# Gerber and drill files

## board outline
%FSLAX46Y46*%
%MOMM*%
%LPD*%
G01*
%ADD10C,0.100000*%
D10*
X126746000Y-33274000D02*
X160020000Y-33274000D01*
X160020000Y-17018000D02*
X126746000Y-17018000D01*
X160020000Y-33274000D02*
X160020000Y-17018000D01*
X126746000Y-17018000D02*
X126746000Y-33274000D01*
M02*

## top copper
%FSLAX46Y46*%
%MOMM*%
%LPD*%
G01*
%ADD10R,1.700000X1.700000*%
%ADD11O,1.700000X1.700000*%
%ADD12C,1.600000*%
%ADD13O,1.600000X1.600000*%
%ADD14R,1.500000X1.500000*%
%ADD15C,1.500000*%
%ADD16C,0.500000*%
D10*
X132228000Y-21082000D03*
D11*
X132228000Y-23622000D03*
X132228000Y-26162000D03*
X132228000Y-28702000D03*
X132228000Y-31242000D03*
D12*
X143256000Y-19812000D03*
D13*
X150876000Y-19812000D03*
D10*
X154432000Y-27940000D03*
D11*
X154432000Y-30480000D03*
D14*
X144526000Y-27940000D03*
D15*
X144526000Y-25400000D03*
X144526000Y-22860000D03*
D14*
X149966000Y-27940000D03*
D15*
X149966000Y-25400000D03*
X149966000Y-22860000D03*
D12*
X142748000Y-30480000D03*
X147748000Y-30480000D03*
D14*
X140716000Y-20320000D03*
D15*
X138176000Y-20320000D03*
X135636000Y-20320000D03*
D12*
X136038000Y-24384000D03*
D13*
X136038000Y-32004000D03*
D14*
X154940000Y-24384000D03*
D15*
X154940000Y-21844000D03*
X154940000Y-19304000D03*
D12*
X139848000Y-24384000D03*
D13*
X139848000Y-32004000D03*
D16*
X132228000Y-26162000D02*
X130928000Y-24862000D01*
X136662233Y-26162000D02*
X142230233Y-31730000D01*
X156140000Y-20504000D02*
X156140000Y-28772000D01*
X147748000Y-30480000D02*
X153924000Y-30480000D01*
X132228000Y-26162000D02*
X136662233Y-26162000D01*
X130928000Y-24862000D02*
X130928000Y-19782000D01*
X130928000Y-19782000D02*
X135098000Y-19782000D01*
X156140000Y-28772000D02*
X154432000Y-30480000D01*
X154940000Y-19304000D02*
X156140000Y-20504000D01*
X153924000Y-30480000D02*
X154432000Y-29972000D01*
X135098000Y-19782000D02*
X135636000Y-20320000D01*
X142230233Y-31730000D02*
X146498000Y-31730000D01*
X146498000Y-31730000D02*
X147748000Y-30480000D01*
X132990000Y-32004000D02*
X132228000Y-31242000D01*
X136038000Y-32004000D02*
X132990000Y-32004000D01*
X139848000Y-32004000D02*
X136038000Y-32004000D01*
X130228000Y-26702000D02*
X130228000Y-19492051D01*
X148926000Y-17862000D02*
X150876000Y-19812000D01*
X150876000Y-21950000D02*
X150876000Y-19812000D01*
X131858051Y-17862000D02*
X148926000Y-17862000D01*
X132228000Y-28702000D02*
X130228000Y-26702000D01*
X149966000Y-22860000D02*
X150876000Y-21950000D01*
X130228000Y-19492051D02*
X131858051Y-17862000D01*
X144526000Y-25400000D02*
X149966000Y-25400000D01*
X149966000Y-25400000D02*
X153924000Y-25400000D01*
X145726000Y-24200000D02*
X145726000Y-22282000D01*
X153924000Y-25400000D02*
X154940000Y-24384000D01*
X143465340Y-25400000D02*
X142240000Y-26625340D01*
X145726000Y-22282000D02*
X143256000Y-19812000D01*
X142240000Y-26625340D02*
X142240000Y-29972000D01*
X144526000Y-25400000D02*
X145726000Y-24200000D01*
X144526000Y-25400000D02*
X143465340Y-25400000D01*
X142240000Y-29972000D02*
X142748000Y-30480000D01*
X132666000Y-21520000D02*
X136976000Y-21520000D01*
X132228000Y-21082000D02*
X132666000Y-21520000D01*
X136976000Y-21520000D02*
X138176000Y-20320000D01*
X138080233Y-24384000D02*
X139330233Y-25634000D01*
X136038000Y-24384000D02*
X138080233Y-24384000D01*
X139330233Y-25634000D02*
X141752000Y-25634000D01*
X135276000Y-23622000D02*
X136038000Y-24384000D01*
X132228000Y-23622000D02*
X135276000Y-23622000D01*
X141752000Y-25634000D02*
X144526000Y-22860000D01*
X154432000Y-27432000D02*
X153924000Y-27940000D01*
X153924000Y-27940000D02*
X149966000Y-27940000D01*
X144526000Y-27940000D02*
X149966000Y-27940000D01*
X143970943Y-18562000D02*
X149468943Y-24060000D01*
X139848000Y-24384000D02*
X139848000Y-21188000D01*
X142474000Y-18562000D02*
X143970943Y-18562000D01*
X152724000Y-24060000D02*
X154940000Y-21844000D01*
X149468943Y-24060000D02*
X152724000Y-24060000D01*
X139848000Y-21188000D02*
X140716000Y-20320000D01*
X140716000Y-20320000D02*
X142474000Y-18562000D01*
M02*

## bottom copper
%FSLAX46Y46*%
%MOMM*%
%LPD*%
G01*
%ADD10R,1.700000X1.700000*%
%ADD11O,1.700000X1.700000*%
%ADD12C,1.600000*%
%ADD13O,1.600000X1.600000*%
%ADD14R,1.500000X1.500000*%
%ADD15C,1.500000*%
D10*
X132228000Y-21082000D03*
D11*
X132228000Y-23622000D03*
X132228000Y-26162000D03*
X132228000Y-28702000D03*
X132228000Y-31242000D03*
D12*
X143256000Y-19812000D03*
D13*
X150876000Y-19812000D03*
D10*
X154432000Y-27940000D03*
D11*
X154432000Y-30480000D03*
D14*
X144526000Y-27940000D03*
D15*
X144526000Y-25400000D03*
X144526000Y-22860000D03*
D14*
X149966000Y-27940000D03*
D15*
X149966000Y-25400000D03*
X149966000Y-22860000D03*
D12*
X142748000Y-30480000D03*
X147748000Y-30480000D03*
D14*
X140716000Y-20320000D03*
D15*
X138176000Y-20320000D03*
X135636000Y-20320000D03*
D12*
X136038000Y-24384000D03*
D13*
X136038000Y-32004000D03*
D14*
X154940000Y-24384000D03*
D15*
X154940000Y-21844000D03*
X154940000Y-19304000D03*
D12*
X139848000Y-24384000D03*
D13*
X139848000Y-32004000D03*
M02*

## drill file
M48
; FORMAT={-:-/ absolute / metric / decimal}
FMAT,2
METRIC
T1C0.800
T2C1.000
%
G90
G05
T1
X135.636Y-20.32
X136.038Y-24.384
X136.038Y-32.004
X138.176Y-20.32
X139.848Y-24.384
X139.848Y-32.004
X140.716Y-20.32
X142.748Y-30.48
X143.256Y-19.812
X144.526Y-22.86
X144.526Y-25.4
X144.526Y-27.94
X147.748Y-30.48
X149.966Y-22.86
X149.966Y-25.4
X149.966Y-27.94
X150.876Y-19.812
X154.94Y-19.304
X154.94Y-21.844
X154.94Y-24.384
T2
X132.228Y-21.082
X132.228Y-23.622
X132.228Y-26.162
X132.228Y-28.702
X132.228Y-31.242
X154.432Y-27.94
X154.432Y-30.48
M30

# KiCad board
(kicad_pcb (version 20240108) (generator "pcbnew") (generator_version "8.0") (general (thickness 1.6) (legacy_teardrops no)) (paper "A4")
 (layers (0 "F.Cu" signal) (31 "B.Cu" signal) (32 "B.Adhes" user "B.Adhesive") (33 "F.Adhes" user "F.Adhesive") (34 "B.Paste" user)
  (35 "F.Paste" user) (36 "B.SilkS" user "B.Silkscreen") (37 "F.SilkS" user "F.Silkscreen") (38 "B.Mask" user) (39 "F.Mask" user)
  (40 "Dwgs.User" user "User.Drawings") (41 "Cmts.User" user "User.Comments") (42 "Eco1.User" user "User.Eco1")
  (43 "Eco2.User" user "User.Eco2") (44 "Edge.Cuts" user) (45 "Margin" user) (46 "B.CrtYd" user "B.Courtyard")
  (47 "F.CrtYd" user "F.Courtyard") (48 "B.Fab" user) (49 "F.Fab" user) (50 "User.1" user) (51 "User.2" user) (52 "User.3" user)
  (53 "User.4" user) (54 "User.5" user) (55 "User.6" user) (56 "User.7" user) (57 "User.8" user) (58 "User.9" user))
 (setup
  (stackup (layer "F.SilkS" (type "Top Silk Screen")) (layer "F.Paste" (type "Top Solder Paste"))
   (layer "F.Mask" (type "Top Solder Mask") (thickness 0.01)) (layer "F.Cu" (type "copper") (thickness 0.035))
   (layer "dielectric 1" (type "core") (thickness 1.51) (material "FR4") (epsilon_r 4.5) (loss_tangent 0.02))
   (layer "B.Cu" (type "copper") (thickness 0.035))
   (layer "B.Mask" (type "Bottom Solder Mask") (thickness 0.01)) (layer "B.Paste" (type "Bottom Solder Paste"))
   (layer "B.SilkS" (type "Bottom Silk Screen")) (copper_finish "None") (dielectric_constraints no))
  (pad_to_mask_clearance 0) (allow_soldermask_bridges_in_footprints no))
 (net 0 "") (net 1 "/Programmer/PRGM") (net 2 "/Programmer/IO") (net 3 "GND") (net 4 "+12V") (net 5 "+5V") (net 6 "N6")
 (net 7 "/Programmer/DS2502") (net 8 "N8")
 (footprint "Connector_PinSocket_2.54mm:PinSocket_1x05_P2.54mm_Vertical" (layer "F.Cu") (at 132.228 21.082)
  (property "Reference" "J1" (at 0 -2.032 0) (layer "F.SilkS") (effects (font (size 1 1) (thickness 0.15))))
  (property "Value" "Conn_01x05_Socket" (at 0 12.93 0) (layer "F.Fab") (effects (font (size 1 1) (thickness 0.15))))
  (pad "1" thru_hole rect (at 0 0) (size 1.7 1.7) (drill 1) (layers "*.Cu" "*.Mask") (remove_unused_layers no) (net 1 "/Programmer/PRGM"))
  (pad "2" thru_hole oval (at 0 2.54) (size 1.7 1.7) (drill 1) (layers "*.Cu" "*.Mask") (remove_unused_layers no) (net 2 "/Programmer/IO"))
  (pad "3" thru_hole oval (at 0 5.08) (size 1.7 1.7) (drill 1) (layers "*.Cu" "*.Mask") (remove_unused_layers no) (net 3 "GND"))
  (pad "4" thru_hole oval (at 0 7.62) (size 1.7 1.7) (drill 1) (layers "*.Cu" "*.Mask") (remove_unused_layers no) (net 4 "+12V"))
  (pad "5" thru_hole oval (at 0 10.16) (size 1.7 1.7) (drill 1) (layers "*.Cu" "*.Mask") (remove_unused_layers no) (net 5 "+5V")))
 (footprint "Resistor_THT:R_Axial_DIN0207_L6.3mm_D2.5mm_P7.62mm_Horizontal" (layer "F.Cu") (at 143.256 19.812)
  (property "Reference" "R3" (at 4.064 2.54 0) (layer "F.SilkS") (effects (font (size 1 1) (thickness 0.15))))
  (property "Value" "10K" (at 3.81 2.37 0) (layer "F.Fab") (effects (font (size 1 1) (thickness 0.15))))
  (pad "1" thru_hole circle (at 0 0) (size 1.6 1.6) (drill 0.8) (layers "*.Cu" "*.Mask") (remove_unused_layers no) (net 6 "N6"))
  (pad "2" thru_hole oval (at 7.62 0) (size 1.6 1.6) (drill 0.8) (layers "*.Cu" "*.Mask") (remove_unused_layers no) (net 4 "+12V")))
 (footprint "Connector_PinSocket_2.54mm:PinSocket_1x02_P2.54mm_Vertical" (layer "F.Cu") (at 154.432 27.94)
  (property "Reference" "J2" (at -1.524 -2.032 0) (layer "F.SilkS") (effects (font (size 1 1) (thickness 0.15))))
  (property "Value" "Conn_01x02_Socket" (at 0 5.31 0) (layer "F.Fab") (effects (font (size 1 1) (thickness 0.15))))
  (pad "1" thru_hole rect (at 0 0) (size 1.7 1.7) (drill 1) (layers "*.Cu" "*.Mask") (remove_unused_layers no) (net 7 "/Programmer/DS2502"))
  (pad "2" thru_hole oval (at 0 2.54) (size 1.7 1.7) (drill 1) (layers "*.Cu" "*.Mask") (remove_unused_layers no) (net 3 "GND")))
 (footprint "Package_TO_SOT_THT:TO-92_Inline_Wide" (layer "F.Cu") (at 144.526 27.94 90)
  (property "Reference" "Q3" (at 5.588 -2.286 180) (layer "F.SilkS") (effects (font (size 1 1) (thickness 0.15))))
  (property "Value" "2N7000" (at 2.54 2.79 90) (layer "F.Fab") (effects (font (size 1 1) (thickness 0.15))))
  (pad "1" thru_hole rect (at 0 0 90) (size 1.5 1.5) (drill 0.8) (layers "*.Cu" "*.Mask") (remove_unused_layers no)
   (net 7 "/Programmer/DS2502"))
  (pad "2" thru_hole circle (at 2.54 0 90) (size 1.5 1.5) (drill 0.8) (layers "*.Cu" "*.Mask") (remove_unused_layers no) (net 6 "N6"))
  (pad "3" thru_hole circle (at 5.08 0 90) (size 1.5 1.5) (drill 0.8) (layers "*.Cu" "*.Mask") (remove_unused_layers no)
   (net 2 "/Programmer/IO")))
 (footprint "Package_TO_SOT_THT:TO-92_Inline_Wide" (layer "F.Cu") (at 149.966 27.94 90)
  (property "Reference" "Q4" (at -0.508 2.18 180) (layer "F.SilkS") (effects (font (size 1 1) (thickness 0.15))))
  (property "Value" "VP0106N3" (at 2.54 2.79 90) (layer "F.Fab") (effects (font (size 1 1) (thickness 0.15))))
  (pad "1" thru_hole rect (at 0 0 90) (size 1.5 1.5) (drill 0.8) (layers "*.Cu" "*.Mask") (remove_unused_layers no)
   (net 7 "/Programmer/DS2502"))
  (pad "2" thru_hole circle (at 2.54 0 90) (size 1.5 1.5) (drill 0.8) (layers "*.Cu" "*.Mask") (remove_unused_layers no) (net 6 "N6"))
  (pad "3" thru_hole circle (at 5.08 0 90) (size 1.5 1.5) (drill 0.8) (layers "*.Cu" "*.Mask") (remove_unused_layers no) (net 4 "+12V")))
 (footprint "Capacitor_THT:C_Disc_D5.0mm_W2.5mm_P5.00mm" (layer "F.Cu") (at 142.748 30.48)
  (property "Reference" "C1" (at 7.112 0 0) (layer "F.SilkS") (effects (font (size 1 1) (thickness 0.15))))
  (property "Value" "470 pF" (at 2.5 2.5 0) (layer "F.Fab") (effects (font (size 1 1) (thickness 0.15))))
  (pad "1" thru_hole circle (at 0 0) (size 1.6 1.6) (drill 0.8) (layers "*.Cu" "*.Mask") (remove_unused_layers no) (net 6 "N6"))
  (pad "2" thru_hole circle (at 5 0) (size 1.6 1.6) (drill 0.8) (layers "*.Cu" "*.Mask") (remove_unused_layers no) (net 3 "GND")))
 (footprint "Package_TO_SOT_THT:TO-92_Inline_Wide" (layer "F.Cu") (at 140.716 20.32 180)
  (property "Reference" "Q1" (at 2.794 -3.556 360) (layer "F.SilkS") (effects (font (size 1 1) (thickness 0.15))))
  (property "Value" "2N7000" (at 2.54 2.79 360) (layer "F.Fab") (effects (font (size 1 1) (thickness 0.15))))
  (pad "1" thru_hole rect (at 0 0 180) (size 1.5 1.5) (drill 0.8) (layers "*.Cu" "*.Mask") (remove_unused_layers no) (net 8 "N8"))
  (pad "2" thru_hole circle (at 2.54 0 180) (size 1.5 1.5) (drill 0.8) (layers "*.Cu" "*.Mask") (remove_unused_layers no)
   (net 1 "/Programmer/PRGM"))
  (pad "3" thru_hole circle (at 5.08 0 180) (size 1.5 1.5) (drill 0.8) (layers "*.Cu" "*.Mask") (remove_unused_layers no) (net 3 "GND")))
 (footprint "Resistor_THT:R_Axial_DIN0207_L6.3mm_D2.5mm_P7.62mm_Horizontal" (layer "F.Cu") (at 136.038 24.384 -90)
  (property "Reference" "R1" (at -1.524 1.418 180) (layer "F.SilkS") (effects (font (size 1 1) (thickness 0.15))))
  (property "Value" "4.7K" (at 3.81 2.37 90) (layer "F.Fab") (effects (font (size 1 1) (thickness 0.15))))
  (pad "1" thru_hole circle (at 0 0 270) (size 1.6 1.6) (drill 0.8) (layers "*.Cu" "*.Mask") (remove_unused_layers no)
   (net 2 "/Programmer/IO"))
  (pad "2" thru_hole oval (at 7.62 0 270) (size 1.6 1.6) (drill 0.8) (layers "*.Cu" "*.Mask") (remove_unused_layers no) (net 5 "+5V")))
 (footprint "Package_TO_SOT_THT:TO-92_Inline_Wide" (layer "F.Cu") (at 154.94 24.384 90)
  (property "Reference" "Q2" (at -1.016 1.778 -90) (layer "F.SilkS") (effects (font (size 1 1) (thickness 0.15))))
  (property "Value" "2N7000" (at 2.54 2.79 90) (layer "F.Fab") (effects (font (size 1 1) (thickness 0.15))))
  (pad "1" thru_hole rect (at 0 0 90) (size 1.5 1.5) (drill 0.8) (layers "*.Cu" "*.Mask") (remove_unused_layers no) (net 6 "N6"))
  (pad "2" thru_hole circle (at 2.54 0 90) (size 1.5 1.5) (drill 0.8) (layers "*.Cu" "*.Mask") (remove_unused_layers no) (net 8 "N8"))
  (pad "3" thru_hole circle (at 5.08 0 90) (size 1.5 1.5) (drill 0.8) (layers "*.Cu" "*.Mask") (remove_unused_layers no) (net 3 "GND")))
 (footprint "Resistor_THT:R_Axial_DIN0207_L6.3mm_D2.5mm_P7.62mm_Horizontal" (layer "F.Cu") (at 139.848 24.384 -90)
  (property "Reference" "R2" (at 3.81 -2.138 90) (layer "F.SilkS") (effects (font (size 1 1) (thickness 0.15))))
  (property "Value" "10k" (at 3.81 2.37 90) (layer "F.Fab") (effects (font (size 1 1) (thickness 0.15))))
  (pad "1" thru_hole circle (at 0 0 270) (size 1.6 1.6) (drill 0.8) (layers "*.Cu" "*.Mask") (remove_unused_layers no) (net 8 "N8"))
  (pad "2" thru_hole oval (at 7.62 0 270) (size 1.6 1.6) (drill 0.8) (layers "*.Cu" "*.Mask") (remove_unused_layers no) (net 5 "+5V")))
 (gr_line (start 126.746 33.274) (end 160.02 33.274) (stroke (width 0.1) (type default)) (layer "Edge.Cuts"))
 (gr_line (start 160.02 17.018) (end 126.746 17.018) (stroke (width 0.1) (type default)) (layer "Edge.Cuts"))
 (gr_line (start 160.02 33.274) (end 160.02 17.018) (stroke (width 0.1) (type default)) (layer "Edge.Cuts"))
 (gr_line (start 126.746 17.018) (end 126.746 33.274) (stroke (width 0.1) (type default)) (layer "Edge.Cuts"))
 (segment (start 132.228 26.162) (end 130.928 24.862) (width 0.5) (layer "F.Cu") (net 3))
 (segment (start 136.662233 26.162) (end 142.230233 31.73) (width 0.5) (layer "F.Cu") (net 3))
 (segment (start 156.14 20.504) (end 156.14 28.772) (width 0.5) (layer "F.Cu") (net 3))
 (segment (start 147.748 30.48) (end 153.924 30.48) (width 0.5) (layer "F.Cu") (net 3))
 (segment (start 132.228 26.162) (end 136.662233 26.162) (width 0.5) (layer "F.Cu") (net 3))
 (segment (start 130.928 24.862) (end 130.928 19.782) (width 0.5) (layer "F.Cu") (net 3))
 (segment (start 130.928 19.782) (end 135.098 19.782) (width 0.5) (layer "F.Cu") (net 3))
 (segment (start 156.14 28.772) (end 154.432 30.48) (width 0.5) (layer "F.Cu") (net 3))
 (segment (start 154.94 19.304) (end 156.14 20.504) (width 0.5) (layer "F.Cu") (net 3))
 (segment (start 153.924 30.48) (end 154.432 29.972) (width 0.5) (layer "F.Cu") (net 3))
 (segment (start 135.098 19.782) (end 135.636 20.32) (width 0.5) (layer "F.Cu") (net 3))
 (segment (start 142.230233 31.73) (end 146.498 31.73) (width 0.5) (layer "F.Cu") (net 3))
 (segment (start 146.498 31.73) (end 147.748 30.48) (width 0.5) (layer "F.Cu") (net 3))
 (segment (start 132.99 32.004) (end 132.228 31.242) (width 0.5) (layer "F.Cu") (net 5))
 (segment (start 136.038 32.004) (end 132.99 32.004) (width 0.5) (layer "F.Cu") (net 5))
 (segment (start 139.848 32.004) (end 136.038 32.004) (width 0.5) (layer "F.Cu") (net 5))
 (segment (start 130.228 26.702) (end 130.228 19.492051) (width 0.5) (layer "F.Cu") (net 4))
 (segment (start 148.926 17.862) (end 150.876 19.812) (width 0.5) (layer "F.Cu") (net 4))
 (segment (start 150.876 21.95) (end 150.876 19.812) (width 0.5) (layer "F.Cu") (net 4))
 (segment (start 131.858051 17.862) (end 148.926 17.862) (width 0.5) (layer "F.Cu") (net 4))
 (segment (start 132.228 28.702) (end 130.228 26.702) (width 0.5) (layer "F.Cu") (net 4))
 (segment (start 149.966 22.86) (end 150.876 21.95) (width 0.5) (layer "F.Cu") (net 4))
 (segment (start 130.228 19.492051) (end 131.858051 17.862) (width 0.5) (layer "F.Cu") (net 4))
 (segment (start 144.526 25.4) (end 149.966 25.4) (width 0.5) (layer "F.Cu") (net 6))
 (segment (start 149.966 25.4) (end 153.924 25.4) (width 0.5) (layer "F.Cu") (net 6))
 (segment (start 145.726 24.2) (end 145.726 22.282) (width 0.5) (layer "F.Cu") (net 6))
 (segment (start 153.924 25.4) (end 154.94 24.384) (width 0.5) (layer "F.Cu") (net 6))
 (segment (start 143.46534 25.4) (end 142.24 26.62534) (width 0.5) (layer "F.Cu") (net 6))
 (segment (start 145.726 22.282) (end 143.256 19.812) (width 0.5) (layer "F.Cu") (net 6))
 (segment (start 142.24 26.62534) (end 142.24 29.972) (width 0.5) (layer "F.Cu") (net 6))
 (segment (start 144.526 25.4) (end 145.726 24.2) (width 0.5) (layer "F.Cu") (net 6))
 (segment (start 144.526 25.4) (end 143.46534 25.4) (width 0.5) (layer "F.Cu") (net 6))
 (segment (start 142.24 29.972) (end 142.748 30.48) (width 0.5) (layer "F.Cu") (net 6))
 (segment (start 132.666 21.52) (end 136.976 21.52) (width 0.5) (layer "F.Cu") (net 1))
 (segment (start 132.228 21.082) (end 132.666 21.52) (width 0.5) (layer "F.Cu") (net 1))
 (segment (start 136.976 21.52) (end 138.176 20.32) (width 0.5) (layer "F.Cu") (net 1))
 (segment (start 138.080233 24.384) (end 139.330233 25.634) (width 0.5) (layer "F.Cu") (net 2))
 (segment (start 136.038 24.384) (end 138.080233 24.384) (width 0.5) (layer "F.Cu") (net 2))
 (segment (start 139.330233 25.634) (end 141.752 25.634) (width 0.5) (layer "F.Cu") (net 2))
 (segment (start 135.276 23.622) (end 136.038 24.384) (width 0.5) (layer "F.Cu") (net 2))
 (segment (start 132.228 23.622) (end 135.276 23.622) (width 0.5) (layer "F.Cu") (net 2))
 (segment (start 141.752 25.634) (end 144.526 22.86) (width 0.5) (layer "F.Cu") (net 2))
 (segment (start 154.432 27.432) (end 153.924 27.94) (width 0.5) (layer "F.Cu") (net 7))
 (segment (start 153.924 27.94) (end 149.966 27.94) (width 0.5) (layer "F.Cu") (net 7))
 (segment (start 144.526 27.94) (end 149.966 27.94) (width 0.5) (layer "F.Cu") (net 7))
 (segment (start 143.970943 18.562) (end 149.468943 24.06) (width 0.5) (layer "F.Cu") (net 8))
 (segment (start 139.848 24.384) (end 139.848 21.188) (width 0.5) (layer "F.Cu") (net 8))
 (segment (start 142.474 18.562) (end 143.970943 18.562) (width 0.5) (layer "F.Cu") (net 8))
 (segment (start 152.724 24.06) (end 154.94 21.844) (width 0.5) (layer "F.Cu") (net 8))
 (segment (start 149.468943 24.06) (end 152.724 24.06) (width 0.5) (layer "F.Cu") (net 8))
 (segment (start 139.848 21.188) (end 140.716 20.32) (width 0.5) (layer "F.Cu") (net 8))
 (segment (start 140.716 20.32) (end 142.474 18.562) (width 0.5) (layer "F.Cu") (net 8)))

